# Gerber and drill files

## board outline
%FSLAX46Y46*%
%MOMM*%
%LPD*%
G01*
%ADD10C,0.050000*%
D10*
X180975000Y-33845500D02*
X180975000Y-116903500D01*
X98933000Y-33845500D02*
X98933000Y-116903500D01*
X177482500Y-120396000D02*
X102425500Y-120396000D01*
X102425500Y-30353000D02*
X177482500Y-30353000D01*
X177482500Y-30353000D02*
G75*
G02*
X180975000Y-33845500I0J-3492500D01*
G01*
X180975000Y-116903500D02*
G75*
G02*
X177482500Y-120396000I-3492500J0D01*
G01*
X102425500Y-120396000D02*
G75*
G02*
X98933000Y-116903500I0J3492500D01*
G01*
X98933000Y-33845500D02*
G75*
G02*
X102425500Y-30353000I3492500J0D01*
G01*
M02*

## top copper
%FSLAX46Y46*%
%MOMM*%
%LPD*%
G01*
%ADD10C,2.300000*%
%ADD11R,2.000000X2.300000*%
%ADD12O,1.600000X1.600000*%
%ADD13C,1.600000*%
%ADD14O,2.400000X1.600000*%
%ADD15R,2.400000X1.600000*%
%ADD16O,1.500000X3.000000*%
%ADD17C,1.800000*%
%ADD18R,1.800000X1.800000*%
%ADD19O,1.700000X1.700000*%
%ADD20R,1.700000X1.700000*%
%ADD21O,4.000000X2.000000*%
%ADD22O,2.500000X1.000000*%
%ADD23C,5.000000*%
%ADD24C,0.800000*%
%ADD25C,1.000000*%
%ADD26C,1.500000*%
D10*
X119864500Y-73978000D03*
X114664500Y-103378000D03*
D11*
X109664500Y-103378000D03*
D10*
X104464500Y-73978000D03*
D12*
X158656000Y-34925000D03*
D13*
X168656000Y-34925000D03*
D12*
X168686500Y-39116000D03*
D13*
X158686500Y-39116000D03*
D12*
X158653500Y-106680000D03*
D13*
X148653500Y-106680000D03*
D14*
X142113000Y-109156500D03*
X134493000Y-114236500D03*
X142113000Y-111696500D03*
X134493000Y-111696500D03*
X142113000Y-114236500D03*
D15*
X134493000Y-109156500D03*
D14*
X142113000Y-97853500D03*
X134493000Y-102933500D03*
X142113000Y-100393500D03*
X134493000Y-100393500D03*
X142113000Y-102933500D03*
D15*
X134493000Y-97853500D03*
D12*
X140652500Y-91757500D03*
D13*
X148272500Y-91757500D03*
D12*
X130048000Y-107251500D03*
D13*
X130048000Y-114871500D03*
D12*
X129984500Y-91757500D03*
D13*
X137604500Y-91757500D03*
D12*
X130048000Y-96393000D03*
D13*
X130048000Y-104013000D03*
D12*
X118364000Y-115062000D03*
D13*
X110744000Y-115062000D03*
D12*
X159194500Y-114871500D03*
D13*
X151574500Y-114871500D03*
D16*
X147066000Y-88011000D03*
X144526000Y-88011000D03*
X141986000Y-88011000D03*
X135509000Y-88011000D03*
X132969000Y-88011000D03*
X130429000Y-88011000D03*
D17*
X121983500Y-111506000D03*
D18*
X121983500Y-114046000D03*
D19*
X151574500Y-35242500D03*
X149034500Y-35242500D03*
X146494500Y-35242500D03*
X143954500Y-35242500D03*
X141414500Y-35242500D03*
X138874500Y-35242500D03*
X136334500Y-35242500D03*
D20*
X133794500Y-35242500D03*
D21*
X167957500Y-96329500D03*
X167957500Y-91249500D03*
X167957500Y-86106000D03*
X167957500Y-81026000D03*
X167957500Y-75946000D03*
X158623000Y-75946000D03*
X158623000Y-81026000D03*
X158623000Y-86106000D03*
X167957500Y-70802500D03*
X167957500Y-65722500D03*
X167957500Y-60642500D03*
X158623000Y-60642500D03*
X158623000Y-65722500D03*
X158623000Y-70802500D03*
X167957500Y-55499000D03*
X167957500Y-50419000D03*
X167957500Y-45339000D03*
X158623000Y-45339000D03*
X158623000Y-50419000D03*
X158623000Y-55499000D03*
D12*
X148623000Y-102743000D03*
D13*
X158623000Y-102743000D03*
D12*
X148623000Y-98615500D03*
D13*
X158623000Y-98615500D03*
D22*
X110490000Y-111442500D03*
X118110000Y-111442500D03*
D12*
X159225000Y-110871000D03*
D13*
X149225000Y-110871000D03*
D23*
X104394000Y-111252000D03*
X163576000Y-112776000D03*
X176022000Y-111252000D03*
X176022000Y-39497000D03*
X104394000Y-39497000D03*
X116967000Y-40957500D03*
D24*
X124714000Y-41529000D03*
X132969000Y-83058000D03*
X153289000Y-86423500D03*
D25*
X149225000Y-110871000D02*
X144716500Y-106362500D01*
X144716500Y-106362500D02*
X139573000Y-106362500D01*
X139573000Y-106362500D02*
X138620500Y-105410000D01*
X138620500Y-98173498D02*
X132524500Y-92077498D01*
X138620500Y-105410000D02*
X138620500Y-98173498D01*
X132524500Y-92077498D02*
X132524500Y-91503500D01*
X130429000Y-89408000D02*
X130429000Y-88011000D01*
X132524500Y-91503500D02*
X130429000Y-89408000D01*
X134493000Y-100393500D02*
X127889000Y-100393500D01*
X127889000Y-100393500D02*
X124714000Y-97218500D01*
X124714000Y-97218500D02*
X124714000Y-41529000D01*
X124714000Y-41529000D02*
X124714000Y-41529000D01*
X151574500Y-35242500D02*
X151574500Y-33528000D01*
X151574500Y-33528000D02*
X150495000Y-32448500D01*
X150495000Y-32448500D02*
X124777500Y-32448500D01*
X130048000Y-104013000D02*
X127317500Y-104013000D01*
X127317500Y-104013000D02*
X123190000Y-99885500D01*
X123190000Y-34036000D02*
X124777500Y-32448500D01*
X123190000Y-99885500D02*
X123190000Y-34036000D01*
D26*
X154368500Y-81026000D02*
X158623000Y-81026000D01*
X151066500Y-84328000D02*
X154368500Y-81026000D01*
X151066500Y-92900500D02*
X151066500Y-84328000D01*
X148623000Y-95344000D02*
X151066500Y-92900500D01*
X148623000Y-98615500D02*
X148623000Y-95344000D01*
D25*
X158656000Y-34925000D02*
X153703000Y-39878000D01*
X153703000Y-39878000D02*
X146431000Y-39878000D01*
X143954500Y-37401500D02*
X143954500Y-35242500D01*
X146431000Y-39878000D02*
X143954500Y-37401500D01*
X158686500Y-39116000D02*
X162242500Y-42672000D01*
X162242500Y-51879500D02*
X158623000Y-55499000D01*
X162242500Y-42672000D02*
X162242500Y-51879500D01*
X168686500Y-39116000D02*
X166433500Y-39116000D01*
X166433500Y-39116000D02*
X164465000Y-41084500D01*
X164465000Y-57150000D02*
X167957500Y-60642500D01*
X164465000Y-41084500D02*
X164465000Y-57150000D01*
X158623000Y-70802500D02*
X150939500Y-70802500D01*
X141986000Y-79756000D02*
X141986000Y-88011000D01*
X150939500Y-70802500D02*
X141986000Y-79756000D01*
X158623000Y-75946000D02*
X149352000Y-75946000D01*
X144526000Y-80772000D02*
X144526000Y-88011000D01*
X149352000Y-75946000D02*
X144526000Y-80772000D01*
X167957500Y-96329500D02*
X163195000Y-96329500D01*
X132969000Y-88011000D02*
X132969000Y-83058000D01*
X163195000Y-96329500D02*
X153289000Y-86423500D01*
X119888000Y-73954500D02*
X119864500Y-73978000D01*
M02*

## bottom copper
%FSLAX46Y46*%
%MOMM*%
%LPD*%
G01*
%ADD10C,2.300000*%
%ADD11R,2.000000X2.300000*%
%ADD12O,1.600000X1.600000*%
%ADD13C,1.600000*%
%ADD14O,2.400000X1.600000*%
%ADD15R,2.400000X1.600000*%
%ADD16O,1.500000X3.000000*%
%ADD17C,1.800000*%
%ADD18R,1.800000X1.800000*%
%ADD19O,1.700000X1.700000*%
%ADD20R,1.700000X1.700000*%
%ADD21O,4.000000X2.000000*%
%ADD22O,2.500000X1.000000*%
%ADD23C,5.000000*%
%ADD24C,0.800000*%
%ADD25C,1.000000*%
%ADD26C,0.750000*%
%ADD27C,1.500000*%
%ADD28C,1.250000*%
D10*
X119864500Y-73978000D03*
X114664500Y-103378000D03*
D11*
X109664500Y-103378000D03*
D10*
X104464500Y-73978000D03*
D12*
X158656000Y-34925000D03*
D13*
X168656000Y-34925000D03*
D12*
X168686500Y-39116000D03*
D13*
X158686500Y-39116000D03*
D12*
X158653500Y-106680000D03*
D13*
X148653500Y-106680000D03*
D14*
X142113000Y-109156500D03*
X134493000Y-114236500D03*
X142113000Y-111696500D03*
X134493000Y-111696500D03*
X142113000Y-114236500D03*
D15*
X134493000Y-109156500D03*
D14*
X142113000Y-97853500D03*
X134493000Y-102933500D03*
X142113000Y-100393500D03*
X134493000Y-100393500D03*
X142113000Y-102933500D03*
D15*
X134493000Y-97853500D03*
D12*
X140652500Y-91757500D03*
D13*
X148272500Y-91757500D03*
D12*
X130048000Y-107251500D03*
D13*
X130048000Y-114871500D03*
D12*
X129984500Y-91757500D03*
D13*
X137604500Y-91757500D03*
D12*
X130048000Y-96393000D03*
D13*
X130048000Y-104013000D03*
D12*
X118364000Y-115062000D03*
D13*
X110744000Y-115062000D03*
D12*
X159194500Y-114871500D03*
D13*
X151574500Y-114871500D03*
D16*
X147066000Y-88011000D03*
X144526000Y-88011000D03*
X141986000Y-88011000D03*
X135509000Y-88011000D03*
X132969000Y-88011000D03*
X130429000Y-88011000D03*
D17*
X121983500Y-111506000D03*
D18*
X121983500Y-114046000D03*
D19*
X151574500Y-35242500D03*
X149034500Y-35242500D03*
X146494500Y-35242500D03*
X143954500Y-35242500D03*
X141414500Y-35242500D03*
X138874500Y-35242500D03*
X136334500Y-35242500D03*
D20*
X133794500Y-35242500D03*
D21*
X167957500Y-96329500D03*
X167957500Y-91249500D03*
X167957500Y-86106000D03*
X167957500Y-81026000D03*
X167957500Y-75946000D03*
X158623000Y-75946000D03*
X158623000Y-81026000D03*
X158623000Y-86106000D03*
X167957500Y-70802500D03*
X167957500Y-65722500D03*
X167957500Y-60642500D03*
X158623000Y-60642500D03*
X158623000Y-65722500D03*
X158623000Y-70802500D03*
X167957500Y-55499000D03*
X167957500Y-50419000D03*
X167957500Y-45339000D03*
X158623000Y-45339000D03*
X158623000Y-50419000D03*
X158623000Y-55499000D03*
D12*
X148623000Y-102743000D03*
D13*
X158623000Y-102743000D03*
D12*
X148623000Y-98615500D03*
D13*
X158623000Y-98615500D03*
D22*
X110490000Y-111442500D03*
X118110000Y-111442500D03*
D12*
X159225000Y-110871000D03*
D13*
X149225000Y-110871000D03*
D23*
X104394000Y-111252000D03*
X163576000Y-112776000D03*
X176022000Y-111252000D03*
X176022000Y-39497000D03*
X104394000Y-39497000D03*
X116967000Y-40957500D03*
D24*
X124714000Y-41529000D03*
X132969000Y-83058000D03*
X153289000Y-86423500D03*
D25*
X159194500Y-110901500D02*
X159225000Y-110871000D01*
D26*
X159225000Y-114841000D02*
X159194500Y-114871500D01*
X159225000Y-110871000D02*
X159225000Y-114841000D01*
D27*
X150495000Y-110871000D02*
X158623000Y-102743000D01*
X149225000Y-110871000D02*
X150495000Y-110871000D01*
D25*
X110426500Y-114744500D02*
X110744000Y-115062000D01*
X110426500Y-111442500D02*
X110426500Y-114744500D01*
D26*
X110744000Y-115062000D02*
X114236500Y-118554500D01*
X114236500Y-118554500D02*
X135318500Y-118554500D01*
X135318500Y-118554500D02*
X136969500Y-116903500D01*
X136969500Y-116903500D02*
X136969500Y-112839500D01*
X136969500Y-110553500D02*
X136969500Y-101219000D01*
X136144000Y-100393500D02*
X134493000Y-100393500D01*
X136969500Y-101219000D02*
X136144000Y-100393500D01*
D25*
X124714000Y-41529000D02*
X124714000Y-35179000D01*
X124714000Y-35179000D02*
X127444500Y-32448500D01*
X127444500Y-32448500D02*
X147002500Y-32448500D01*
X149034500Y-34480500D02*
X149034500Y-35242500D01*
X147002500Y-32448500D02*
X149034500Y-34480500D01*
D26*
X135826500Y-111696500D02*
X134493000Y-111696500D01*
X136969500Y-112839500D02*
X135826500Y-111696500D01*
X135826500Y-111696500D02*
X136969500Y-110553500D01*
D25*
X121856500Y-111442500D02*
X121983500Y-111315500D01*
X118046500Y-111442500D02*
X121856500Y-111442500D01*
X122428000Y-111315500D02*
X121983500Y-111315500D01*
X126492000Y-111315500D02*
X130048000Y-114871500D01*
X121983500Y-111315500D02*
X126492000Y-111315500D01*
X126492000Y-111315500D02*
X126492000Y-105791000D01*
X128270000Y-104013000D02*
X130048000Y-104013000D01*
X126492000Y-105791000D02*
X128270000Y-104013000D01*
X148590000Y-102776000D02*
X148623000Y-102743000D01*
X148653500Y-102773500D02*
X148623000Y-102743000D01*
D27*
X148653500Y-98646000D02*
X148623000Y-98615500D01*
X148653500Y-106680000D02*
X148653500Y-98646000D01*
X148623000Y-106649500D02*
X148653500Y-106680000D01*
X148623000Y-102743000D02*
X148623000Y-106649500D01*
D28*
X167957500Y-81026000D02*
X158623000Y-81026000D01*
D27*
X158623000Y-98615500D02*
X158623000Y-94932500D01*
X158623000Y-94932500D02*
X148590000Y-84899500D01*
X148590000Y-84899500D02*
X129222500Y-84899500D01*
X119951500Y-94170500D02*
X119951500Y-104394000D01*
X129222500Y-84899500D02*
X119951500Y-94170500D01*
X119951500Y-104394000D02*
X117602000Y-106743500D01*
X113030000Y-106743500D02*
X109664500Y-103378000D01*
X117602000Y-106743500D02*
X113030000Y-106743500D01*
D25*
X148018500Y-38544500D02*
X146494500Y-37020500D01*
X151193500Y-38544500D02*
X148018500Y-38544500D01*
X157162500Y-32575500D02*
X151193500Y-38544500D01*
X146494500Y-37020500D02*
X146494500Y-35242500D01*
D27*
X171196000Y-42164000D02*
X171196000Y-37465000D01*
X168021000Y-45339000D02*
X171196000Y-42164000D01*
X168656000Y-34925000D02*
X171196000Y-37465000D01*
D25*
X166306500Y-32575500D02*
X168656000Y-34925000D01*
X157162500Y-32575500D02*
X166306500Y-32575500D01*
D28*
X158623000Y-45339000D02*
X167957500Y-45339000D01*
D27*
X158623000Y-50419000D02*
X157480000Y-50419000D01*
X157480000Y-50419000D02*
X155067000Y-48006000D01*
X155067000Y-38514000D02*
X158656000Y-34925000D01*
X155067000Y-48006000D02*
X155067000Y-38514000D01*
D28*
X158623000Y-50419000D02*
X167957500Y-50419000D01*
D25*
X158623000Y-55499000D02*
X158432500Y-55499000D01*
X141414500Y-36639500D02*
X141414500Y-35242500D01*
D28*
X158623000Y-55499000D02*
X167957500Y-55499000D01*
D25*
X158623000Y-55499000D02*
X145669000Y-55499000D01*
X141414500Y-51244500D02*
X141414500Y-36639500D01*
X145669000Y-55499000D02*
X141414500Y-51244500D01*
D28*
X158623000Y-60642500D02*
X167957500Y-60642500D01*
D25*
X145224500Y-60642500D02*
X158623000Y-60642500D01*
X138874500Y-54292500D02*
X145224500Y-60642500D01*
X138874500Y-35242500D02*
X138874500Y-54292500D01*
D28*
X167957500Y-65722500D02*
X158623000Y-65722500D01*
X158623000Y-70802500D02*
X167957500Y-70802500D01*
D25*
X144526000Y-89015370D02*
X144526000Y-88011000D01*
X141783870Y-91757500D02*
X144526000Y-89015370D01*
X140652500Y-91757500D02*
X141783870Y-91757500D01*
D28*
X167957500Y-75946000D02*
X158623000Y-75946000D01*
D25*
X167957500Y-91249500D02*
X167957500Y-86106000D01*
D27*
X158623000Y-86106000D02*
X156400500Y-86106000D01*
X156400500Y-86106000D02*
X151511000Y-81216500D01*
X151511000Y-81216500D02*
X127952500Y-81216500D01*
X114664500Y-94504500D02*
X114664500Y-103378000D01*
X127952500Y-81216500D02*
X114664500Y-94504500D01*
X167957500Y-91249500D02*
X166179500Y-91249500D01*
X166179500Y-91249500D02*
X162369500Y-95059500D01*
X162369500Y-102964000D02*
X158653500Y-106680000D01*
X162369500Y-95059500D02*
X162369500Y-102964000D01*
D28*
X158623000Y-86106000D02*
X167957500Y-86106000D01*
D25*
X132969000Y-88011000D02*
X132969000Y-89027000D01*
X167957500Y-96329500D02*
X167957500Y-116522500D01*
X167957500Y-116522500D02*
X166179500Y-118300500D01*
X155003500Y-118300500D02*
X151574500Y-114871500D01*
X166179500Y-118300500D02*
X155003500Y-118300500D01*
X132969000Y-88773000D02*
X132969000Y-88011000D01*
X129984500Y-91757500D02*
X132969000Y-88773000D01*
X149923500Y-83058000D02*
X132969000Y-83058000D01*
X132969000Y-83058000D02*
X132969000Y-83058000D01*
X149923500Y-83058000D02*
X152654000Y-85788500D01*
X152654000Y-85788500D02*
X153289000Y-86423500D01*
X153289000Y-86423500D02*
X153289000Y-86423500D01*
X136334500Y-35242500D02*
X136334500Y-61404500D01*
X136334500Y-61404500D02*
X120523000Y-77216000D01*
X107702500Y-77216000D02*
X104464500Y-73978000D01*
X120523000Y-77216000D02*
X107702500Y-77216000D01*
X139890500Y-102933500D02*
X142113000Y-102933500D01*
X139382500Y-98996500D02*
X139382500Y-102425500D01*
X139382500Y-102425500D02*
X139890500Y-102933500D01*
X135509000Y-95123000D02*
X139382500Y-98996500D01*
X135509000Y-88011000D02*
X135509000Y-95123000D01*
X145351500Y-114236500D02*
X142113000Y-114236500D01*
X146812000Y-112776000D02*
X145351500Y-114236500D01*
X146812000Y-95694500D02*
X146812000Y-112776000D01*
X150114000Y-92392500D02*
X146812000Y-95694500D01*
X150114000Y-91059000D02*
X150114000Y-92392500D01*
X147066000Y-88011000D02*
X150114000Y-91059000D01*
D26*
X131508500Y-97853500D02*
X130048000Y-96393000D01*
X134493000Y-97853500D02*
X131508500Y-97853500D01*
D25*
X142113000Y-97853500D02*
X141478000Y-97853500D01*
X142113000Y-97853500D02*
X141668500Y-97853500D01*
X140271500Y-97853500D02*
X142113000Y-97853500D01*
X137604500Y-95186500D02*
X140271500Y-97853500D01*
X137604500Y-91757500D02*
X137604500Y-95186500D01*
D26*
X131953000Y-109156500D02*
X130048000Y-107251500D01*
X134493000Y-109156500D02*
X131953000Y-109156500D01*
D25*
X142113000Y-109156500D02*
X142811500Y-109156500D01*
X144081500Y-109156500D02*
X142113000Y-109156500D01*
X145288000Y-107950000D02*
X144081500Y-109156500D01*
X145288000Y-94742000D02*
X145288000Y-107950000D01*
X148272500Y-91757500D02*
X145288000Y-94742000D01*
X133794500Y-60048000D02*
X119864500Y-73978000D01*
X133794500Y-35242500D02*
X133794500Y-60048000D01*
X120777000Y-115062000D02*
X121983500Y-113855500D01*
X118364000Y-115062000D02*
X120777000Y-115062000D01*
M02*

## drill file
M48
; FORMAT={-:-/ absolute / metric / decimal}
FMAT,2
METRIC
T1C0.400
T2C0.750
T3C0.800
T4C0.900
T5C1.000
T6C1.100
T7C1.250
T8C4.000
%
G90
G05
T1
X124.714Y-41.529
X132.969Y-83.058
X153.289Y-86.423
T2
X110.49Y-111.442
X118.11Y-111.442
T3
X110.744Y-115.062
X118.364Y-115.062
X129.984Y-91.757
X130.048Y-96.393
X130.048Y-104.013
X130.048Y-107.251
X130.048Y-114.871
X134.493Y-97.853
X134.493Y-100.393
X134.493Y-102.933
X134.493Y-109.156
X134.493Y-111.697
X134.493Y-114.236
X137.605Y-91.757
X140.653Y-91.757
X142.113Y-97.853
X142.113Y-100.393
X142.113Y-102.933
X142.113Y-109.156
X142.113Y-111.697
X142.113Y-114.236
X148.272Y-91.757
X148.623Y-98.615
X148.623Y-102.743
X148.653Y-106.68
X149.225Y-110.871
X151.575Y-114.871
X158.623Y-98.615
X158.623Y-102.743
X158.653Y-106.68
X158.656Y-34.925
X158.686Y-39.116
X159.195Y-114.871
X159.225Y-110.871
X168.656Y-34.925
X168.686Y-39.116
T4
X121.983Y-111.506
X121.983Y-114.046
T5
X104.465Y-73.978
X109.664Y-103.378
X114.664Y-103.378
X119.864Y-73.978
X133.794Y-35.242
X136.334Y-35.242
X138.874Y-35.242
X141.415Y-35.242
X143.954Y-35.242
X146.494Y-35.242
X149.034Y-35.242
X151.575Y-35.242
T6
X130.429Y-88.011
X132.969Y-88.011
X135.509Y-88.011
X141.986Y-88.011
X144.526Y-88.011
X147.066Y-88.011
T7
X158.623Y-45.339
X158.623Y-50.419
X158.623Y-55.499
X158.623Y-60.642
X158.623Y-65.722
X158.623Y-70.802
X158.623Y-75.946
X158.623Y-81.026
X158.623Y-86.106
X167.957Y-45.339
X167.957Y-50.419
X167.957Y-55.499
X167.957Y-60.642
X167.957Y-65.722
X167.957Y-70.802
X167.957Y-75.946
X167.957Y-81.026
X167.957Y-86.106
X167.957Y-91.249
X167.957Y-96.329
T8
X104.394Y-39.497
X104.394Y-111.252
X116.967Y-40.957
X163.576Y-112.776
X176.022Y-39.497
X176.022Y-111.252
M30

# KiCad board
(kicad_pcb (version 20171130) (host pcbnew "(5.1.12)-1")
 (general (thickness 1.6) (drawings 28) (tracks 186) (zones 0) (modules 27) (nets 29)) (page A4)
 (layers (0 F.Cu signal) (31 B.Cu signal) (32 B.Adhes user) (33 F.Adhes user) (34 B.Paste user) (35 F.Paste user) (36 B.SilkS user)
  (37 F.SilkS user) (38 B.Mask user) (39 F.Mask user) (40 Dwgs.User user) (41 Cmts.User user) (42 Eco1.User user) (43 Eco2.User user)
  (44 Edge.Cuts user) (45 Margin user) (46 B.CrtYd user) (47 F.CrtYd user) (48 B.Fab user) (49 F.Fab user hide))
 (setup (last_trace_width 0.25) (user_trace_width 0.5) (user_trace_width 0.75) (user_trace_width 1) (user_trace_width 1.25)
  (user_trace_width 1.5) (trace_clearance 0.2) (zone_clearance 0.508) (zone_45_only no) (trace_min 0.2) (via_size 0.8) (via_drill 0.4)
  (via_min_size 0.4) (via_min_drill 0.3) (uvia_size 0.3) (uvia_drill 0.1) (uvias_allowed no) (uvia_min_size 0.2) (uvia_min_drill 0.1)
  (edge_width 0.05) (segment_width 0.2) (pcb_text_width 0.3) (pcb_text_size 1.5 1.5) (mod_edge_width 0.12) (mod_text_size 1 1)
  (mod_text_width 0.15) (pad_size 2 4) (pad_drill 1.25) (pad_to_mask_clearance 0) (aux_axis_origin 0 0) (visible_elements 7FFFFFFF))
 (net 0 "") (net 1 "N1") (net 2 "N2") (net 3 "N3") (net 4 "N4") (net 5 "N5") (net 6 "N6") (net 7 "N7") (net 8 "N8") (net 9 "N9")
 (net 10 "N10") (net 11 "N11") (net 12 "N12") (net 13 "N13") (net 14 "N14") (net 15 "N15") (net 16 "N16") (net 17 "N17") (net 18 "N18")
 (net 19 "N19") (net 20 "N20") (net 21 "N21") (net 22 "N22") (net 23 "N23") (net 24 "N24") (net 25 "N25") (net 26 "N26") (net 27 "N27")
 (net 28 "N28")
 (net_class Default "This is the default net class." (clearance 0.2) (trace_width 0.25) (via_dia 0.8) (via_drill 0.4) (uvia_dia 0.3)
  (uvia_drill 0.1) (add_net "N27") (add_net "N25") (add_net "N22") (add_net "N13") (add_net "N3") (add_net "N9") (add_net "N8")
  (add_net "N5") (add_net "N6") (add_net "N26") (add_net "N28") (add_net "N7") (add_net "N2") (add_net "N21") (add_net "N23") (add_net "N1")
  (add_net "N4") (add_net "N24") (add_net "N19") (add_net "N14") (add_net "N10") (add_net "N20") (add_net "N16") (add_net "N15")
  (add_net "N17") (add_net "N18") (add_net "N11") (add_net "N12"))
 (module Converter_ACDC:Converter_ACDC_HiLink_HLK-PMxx (layer F.Cu) (at 109.6645 103.378 90)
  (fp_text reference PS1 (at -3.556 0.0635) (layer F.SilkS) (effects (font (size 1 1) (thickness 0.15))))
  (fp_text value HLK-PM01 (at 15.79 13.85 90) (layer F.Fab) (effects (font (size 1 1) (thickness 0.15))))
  (pad 4 thru_hole circle (at 29.4 10.2 90) (size 2.3 2.3) (drill 1) (layers *.Cu *.Mask) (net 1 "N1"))
  (pad 2 thru_hole circle (at 0 5 90) (size 2.3 2.3) (drill 1) (layers *.Cu *.Mask) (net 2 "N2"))
  (pad 1 thru_hole rect (at 0 0 90) (size 2.3 2) (drill 1) (layers *.Cu *.Mask) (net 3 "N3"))
  (pad 3 thru_hole circle (at 29.4 -5.2 90) (size 2.3 2.3) (drill 1) (layers *.Cu *.Mask) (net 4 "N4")))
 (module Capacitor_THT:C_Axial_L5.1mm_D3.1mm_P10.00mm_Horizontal (layer F.Cu) (at 168.656 34.925 180)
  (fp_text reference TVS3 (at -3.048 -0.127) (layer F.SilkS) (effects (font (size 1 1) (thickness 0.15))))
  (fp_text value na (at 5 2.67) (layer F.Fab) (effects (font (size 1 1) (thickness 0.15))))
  (pad 2 thru_hole oval (at 10 0 180) (size 1.6 1.6) (drill 0.8) (layers *.Cu *.Mask) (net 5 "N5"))
  (pad 1 thru_hole circle (at 0 0 180) (size 1.6 1.6) (drill 0.8) (layers *.Cu *.Mask) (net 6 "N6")))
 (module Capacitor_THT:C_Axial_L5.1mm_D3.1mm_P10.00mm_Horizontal (layer F.Cu) (at 158.6865 39.116)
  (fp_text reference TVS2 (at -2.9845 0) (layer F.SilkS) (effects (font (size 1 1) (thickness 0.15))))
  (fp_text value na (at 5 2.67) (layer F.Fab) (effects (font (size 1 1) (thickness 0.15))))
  (pad 2 thru_hole oval (at 10 0) (size 1.6 1.6) (drill 0.8) (layers *.Cu *.Mask) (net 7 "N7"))
  (pad 1 thru_hole circle (at 0 0) (size 1.6 1.6) (drill 0.8) (layers *.Cu *.Mask) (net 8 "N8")))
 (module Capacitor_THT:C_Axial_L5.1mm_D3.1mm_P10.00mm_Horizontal (layer F.Cu) (at 148.6535 106.68)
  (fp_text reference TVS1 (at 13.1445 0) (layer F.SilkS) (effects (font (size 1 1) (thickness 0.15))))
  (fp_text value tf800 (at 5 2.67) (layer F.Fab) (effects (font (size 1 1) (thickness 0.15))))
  (pad 2 thru_hole oval (at 10 0) (size 1.6 1.6) (drill 0.8) (layers *.Cu *.Mask) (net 2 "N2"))
  (pad 1 thru_hole circle (at 0 0) (size 1.6 1.6) (drill 0.8) (layers *.Cu *.Mask) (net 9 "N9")))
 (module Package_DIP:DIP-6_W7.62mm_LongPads (layer F.Cu) (at 134.493 109.1565)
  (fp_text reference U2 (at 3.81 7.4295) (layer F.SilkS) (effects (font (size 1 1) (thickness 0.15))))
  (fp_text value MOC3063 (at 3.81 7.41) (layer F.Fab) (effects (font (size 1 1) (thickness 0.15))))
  (pad 6 thru_hole oval (at 7.62 0) (size 2.4 1.6) (drill 0.8) (layers *.Cu *.Mask) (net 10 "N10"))
  (pad 3 thru_hole oval (at 0 5.08) (size 2.4 1.6) (drill 0.8) (layers *.Cu *.Mask) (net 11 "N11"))
  (pad 5 thru_hole oval (at 7.62 2.54) (size 2.4 1.6) (drill 0.8) (layers *.Cu *.Mask) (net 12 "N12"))
  (pad 2 thru_hole oval (at 0 2.54) (size 2.4 1.6) (drill 0.8) (layers *.Cu *.Mask) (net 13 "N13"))
  (pad 4 thru_hole oval (at 7.62 5.08) (size 2.4 1.6) (drill 0.8) (layers *.Cu *.Mask) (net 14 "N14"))
  (pad 1 thru_hole rect (at 0 0) (size 2.4 1.6) (drill 0.8) (layers *.Cu *.Mask) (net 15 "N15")))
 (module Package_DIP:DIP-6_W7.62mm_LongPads (layer F.Cu) (at 134.493 97.8535)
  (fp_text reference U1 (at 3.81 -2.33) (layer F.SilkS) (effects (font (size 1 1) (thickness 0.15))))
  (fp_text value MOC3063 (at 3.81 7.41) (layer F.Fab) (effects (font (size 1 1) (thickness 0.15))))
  (pad 6 thru_hole oval (at 7.62 0) (size 2.4 1.6) (drill 0.8) (layers *.Cu *.Mask) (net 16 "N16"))
  (pad 3 thru_hole oval (at 0 5.08) (size 2.4 1.6) (drill 0.8) (layers *.Cu *.Mask) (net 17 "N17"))
  (pad 5 thru_hole oval (at 7.62 2.54) (size 2.4 1.6) (drill 0.8) (layers *.Cu *.Mask) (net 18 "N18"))
  (pad 2 thru_hole oval (at 0 2.54) (size 2.4 1.6) (drill 0.8) (layers *.Cu *.Mask) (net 13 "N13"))
  (pad 4 thru_hole oval (at 7.62 5.08) (size 2.4 1.6) (drill 0.8) (layers *.Cu *.Mask) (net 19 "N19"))
  (pad 1 thru_hole rect (at 0 0) (size 2.4 1.6) (drill 0.8) (layers *.Cu *.Mask) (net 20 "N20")))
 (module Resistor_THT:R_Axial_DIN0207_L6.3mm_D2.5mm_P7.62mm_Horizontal (layer F.Cu) (at 148.2725 91.7575 180)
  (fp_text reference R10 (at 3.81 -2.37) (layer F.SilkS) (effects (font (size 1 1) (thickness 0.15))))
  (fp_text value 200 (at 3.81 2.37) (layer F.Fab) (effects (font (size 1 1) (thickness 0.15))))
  (pad 2 thru_hole oval (at 7.62 0 180) (size 1.6 1.6) (drill 0.8) (layers *.Cu *.Mask) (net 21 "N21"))
  (pad 1 thru_hole circle (at 0 0 180) (size 1.6 1.6) (drill 0.8) (layers *.Cu *.Mask) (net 10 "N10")))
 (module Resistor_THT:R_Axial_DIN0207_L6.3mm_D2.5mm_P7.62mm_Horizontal (layer F.Cu) (at 130.048 114.8715 90)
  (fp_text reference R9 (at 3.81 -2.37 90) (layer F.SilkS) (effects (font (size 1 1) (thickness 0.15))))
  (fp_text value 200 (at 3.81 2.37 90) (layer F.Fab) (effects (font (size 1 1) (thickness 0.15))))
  (pad 2 thru_hole oval (at 7.62 0 90) (size 1.6 1.6) (drill 0.8) (layers *.Cu *.Mask) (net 15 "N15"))
  (pad 1 thru_hole circle (at 0 0 90) (size 1.6 1.6) (drill 0.8) (layers *.Cu *.Mask) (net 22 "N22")))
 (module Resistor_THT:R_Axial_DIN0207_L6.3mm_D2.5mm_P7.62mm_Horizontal (layer F.Cu) (at 137.6045 91.7575 180)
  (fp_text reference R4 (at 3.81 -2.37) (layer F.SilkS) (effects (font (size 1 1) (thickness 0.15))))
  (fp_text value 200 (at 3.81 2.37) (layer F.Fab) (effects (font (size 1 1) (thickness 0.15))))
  (pad 2 thru_hole oval (at 7.62 0 180) (size 1.6 1.6) (drill 0.8) (layers *.Cu *.Mask) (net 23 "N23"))
  (pad 1 thru_hole circle (at 0 0 180) (size 1.6 1.6) (drill 0.8) (layers *.Cu *.Mask) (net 16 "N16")))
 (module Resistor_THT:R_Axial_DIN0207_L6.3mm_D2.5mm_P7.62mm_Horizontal (layer F.Cu) (at 130.048 104.013 90)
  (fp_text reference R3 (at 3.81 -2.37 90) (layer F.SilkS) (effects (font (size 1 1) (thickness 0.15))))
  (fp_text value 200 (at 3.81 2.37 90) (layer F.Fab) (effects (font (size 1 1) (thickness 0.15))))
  (pad 2 thru_hole oval (at 7.62 0 90) (size 1.6 1.6) (drill 0.8) (layers *.Cu *.Mask) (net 20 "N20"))
  (pad 1 thru_hole circle (at 0 0 90) (size 1.6 1.6) (drill 0.8) (layers *.Cu *.Mask) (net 22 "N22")))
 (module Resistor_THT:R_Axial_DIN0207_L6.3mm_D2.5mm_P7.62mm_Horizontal (layer F.Cu) (at 110.744 115.062)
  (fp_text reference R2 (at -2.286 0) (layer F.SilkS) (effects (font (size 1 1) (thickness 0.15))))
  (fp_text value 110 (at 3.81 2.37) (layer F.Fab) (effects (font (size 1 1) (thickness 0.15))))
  (pad 2 thru_hole oval (at 7.62 0) (size 1.6 1.6) (drill 0.8) (layers *.Cu *.Mask) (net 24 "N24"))
  (pad 1 thru_hole circle (at 0 0) (size 1.6 1.6) (drill 0.8) (layers *.Cu *.Mask) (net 13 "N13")))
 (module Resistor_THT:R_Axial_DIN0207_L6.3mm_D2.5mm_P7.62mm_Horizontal (layer F.Cu) (at 151.5745 114.8715)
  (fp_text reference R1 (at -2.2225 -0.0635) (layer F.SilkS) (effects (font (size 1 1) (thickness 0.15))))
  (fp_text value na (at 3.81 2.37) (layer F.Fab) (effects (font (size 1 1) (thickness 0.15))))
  (pad 2 thru_hole oval (at 7.62 0) (size 1.6 1.6) (drill 0.8) (layers *.Cu *.Mask) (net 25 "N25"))
  (pad 1 thru_hole circle (at 0 0) (size 1.6 1.6) (drill 0.8) (layers *.Cu *.Mask) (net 23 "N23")))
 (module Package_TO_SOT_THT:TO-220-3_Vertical (layer F.Cu) (at 141.986 88.011)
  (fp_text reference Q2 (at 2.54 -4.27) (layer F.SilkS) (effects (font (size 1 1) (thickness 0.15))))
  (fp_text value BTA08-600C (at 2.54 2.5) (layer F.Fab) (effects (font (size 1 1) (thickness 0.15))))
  (pad 3 thru_hole oval (at 5.08 0) (size 1.5 3) (drill 1.1) (layers *.Cu *.Mask) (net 14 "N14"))
  (pad 2 thru_hole oval (at 2.54 0) (size 1.5 3) (drill 1.1) (layers *.Cu *.Mask) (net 21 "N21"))
  (pad 1 thru_hole oval (at 0 0) (size 1.5 3) (drill 1.1) (layers *.Cu *.Mask) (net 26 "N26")))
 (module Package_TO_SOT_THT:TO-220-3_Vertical (layer F.Cu) (at 130.429 88.011)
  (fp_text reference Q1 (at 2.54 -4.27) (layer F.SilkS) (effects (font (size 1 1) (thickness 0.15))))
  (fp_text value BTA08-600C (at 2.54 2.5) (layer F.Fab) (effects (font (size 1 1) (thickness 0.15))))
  (pad 3 thru_hole oval (at 5.08 0) (size 1.5 3) (drill 1.1) (layers *.Cu *.Mask) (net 19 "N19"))
  (pad 2 thru_hole oval (at 2.54 0) (size 1.5 3) (drill 1.1) (layers *.Cu *.Mask) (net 23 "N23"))
  (pad 1 thru_hole oval (at 0 0) (size 1.5 3) (drill 1.1) (layers *.Cu *.Mask) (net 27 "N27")))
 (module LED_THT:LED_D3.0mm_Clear (layer F.Cu) (at 121.9835 114.046 90)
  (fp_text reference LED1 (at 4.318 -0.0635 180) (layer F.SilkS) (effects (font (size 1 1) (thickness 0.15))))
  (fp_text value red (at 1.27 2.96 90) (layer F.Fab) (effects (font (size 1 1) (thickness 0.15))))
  (pad 2 thru_hole circle (at 2.54 0 90) (size 1.8 1.8) (drill 0.9) (layers *.Cu *.Mask) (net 22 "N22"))
  (pad 1 thru_hole rect (at 0 0 90) (size 1.8 1.8) (drill 0.9) (layers *.Cu *.Mask) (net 24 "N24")))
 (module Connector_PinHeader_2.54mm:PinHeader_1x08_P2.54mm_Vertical (layer F.Cu) (at 133.7945 35.2425 90)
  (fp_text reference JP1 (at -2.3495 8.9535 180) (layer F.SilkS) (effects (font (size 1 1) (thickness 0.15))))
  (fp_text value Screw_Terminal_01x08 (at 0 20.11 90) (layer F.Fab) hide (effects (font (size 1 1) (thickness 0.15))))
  (pad 8 thru_hole oval (at 0 17.78 90) (size 1.7 1.7) (drill 1) (layers *.Cu *.Mask) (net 22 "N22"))
  (pad 7 thru_hole oval (at 0 15.24 90) (size 1.7 1.7) (drill 1) (layers *.Cu *.Mask) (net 13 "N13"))
  (pad 6 thru_hole oval (at 0 12.7 90) (size 1.7 1.7) (drill 1) (layers *.Cu *.Mask) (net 6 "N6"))
  (pad 5 thru_hole oval (at 0 10.16 90) (size 1.7 1.7) (drill 1) (layers *.Cu *.Mask) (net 5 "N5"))
  (pad 4 thru_hole oval (at 0 7.62 90) (size 1.7 1.7) (drill 1) (layers *.Cu *.Mask) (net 8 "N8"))
  (pad 3 thru_hole oval (at 0 5.08 90) (size 1.7 1.7) (drill 1) (layers *.Cu *.Mask) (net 7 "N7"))
  (pad 2 thru_hole oval (at 0 2.54 90) (size 1.7 1.7) (drill 1) (layers *.Cu *.Mask) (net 4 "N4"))
  (pad 1 thru_hole rect (at 0 0 90) (size 1.7 1.7) (drill 1) (layers *.Cu *.Mask) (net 1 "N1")))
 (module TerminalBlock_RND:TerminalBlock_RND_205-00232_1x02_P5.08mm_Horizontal (layer F.Cu) (at 167.9575 91.2495 270)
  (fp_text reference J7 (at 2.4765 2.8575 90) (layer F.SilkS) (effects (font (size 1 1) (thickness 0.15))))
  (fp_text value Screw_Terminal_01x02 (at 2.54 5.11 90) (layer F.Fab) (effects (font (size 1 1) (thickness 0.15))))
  (pad 2 thru_hole oval (at 5.08 0 270) (size 2 4) (drill 1.25) (layers *.Cu *.Mask) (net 23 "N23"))
  (pad 1 thru_hole oval (at 0 0 270) (size 2 4) (drill 1.25) (layers *.Cu *.Mask) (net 2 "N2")))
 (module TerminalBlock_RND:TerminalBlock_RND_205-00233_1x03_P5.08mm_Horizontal (layer F.Cu) (at 167.9575 75.946 270)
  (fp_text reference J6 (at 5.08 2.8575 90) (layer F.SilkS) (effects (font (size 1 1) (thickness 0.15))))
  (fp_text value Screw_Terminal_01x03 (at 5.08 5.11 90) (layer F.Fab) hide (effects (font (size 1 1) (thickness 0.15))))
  (pad 3 thru_hole oval (at 10.16 0 270) (size 2 4) (drill 1.25) (layers *.Cu *.Mask) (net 2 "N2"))
  (pad 2 thru_hole oval (at 5.08 0 270) (size 2 4) (drill 1.25) (layers *.Cu *.Mask) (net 9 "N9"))
  (pad 1 thru_hole oval (at 0 0 270) (size 2 4) (drill 1.25) (layers *.Cu *.Mask) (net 21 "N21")))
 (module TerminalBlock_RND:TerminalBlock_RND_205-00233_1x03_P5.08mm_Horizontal (layer F.Cu) (at 158.623 86.106 90)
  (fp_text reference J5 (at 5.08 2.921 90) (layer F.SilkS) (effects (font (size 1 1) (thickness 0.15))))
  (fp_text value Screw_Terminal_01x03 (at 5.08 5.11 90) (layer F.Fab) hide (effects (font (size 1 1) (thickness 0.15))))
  (pad 3 thru_hole oval (at 10.16 0 90) (size 2 4) (drill 1.25) (layers *.Cu *.Mask) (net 21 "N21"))
  (pad 2 thru_hole oval (at 5.08 0 90) (size 2 4) (drill 1.25) (layers *.Cu *.Mask) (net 9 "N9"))
  (pad 1 thru_hole oval (at 0 0 90) (size 2 4) (drill 1.25) (layers *.Cu *.Mask) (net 2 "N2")))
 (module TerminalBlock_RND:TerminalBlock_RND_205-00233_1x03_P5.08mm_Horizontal (layer F.Cu) (at 167.9575 60.6425 270)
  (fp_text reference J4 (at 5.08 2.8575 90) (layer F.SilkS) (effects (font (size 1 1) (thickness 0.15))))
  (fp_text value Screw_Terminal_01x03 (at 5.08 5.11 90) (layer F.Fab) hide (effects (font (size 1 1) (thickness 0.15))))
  (pad 3 thru_hole oval (at 10.16 0 270) (size 2 4) (drill 1.25) (layers *.Cu *.Mask) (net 26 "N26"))
  (pad 2 thru_hole oval (at 5.08 0 270) (size 2 4) (drill 1.25) (layers *.Cu *.Mask) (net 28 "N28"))
  (pad 1 thru_hole oval (at 0 0 270) (size 2 4) (drill 1.25) (layers *.Cu *.Mask) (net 7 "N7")))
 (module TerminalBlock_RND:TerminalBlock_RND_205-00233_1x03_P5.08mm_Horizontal (layer F.Cu) (at 158.623 70.8025 90)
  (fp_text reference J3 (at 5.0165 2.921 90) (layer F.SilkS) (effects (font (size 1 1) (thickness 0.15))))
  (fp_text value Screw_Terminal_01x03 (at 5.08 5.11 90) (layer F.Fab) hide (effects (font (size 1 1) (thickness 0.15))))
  (pad 3 thru_hole oval (at 10.16 0 90) (size 2 4) (drill 1.25) (layers *.Cu *.Mask) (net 7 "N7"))
  (pad 2 thru_hole oval (at 5.08 0 90) (size 2 4) (drill 1.25) (layers *.Cu *.Mask) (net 28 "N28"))
  (pad 1 thru_hole oval (at 0 0 90) (size 2 4) (drill 1.25) (layers *.Cu *.Mask) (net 26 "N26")))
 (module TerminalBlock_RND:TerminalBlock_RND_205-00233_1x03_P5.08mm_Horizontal (layer F.Cu) (at 167.9575 45.339 270)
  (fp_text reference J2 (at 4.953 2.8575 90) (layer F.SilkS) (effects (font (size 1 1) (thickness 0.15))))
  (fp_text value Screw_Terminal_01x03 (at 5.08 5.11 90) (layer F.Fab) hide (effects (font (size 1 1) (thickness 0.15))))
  (pad 3 thru_hole oval (at 10.16 0 270) (size 2 4) (drill 1.25) (layers *.Cu *.Mask) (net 8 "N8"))
  (pad 2 thru_hole oval (at 5.08 0 270) (size 2 4) (drill 1.25) (layers *.Cu *.Mask) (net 5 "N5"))
  (pad 1 thru_hole oval (at 0 0 270) (size 2 4) (drill 1.25) (layers *.Cu *.Mask) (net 6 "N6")))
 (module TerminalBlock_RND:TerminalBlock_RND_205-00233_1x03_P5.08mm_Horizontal (layer F.Cu) (at 158.623 55.499 90)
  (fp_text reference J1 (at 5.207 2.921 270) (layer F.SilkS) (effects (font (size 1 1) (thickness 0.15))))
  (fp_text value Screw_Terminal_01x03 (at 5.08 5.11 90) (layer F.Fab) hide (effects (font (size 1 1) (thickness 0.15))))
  (pad 3 thru_hole oval (at 10.16 0 90) (size 2 4) (drill 1.25) (layers *.Cu *.Mask) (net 6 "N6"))
  (pad 2 thru_hole oval (at 5.08 0 90) (size 2 4) (drill 1.25) (layers *.Cu *.Mask) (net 5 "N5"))
  (pad 1 thru_hole oval (at 0 0 90) (size 2 4) (drill 1.25) (layers *.Cu *.Mask) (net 8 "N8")))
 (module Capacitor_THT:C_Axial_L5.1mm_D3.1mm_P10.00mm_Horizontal (layer F.Cu) (at 158.623 102.743 180)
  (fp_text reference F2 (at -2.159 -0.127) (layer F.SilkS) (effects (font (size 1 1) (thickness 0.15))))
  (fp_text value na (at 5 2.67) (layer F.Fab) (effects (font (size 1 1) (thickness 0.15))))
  (pad 2 thru_hole oval (at 10 0 180) (size 1.6 1.6) (drill 0.8) (layers *.Cu *.Mask) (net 9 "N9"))
  (pad 1 thru_hole circle (at 0 0 180) (size 1.6 1.6) (drill 0.8) (layers *.Cu *.Mask) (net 27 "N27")))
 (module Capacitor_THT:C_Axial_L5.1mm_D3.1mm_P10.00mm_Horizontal (layer F.Cu) (at 158.623 98.6155 180)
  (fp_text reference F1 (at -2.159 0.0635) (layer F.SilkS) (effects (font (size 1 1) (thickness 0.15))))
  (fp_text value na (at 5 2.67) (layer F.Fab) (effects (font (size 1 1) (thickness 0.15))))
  (pad 2 thru_hole oval (at 10 0 180) (size 1.6 1.6) (drill 0.8) (layers *.Cu *.Mask) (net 9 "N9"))
  (pad 1 thru_hole circle (at 0 0 180) (size 1.6 1.6) (drill 0.8) (layers *.Cu *.Mask) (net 3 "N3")))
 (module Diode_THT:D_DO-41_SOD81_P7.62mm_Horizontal (layer F.Cu) (at 118.11 111.4425 180)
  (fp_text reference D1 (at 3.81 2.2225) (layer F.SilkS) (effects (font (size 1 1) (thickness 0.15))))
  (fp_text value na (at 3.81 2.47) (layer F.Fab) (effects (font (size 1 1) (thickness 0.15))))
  (pad 2 thru_hole oval (at 7.62 0 180) (size 2.5 1) (drill 0.75) (layers *.Cu *.Mask) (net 13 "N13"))
  (pad 1 thru_hole oval (at 0 0 180) (size 2.5 1) (drill 0.75) (layers *.Cu *.Mask) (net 22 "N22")))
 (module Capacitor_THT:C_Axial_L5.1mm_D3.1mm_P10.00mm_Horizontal (layer F.Cu) (at 149.225 110.871)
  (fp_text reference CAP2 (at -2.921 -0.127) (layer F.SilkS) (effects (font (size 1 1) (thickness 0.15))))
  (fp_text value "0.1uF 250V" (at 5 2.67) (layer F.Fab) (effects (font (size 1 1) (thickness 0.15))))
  (pad 2 thru_hole oval (at 10 0) (size 1.6 1.6) (drill 0.8) (layers *.Cu *.Mask) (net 25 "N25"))
  (pad 1 thru_hole circle (at 0 0) (size 1.6 1.6) (drill 0.8) (layers *.Cu *.Mask) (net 27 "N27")))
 (gr_line (start 180.975 33.8455) (end 180.975 116.9035) (layer Edge.Cuts) (width 0.05))
 (gr_line (start 98.933 33.8455) (end 98.933 116.9035) (layer Edge.Cuts) (width 0.05))
 (gr_line (start 177.4825 120.396) (end 102.4255 120.396) (layer Edge.Cuts) (width 0.05))
 (gr_line (start 102.4255 30.353) (end 177.4825 30.353) (layer Edge.Cuts) (width 0.05))
 (gr_arc (start 177.4825 33.8455) (end 180.975 33.8455) (angle -90) (layer Edge.Cuts) (width 0.05))
 (gr_arc (start 177.4825 116.9035) (end 177.4825 120.396) (angle -90) (layer Edge.Cuts) (width 0.05))
 (gr_arc (start 102.4255 116.9035) (end 98.933 116.9035) (angle -90) (layer Edge.Cuts) (width 0.05))
 (gr_arc (start 102.4255 33.8455) (end 102.4255 30.353) (angle -90) (layer Edge.Cuts) (width 0.05))
 (via (at 104.394 111.252) (size 5) (drill 4) (layers F.Cu B.Cu) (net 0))
 (via (at 163.576 112.776) (size 5) (drill 4) (layers F.Cu B.Cu) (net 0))
 (via (at 176.022 111.252) (size 5) (drill 4) (layers F.Cu B.Cu) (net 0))
 (via (at 176.022 39.497) (size 5) (drill 4) (layers F.Cu B.Cu) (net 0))
 (via (at 104.394 39.497) (size 5) (drill 4) (layers F.Cu B.Cu) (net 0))
 (via (at 116.967 40.9575) (size 5) (drill 4) (layers F.Cu B.Cu) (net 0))
 (segment (start 159.1945 110.9015) (end 159.225 110.871) (width 1) (layer B.Cu) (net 25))
 (segment (start 159.225 114.841) (end 159.1945 114.8715) (width 0.75) (layer B.Cu) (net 25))
 (segment (start 159.225 110.871) (end 159.225 114.841) (width 0.75) (layer B.Cu) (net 25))
 (segment (start 150.495 110.871) (end 158.623 102.743) (width 1.5) (layer B.Cu) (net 27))
 (segment (start 149.225 110.871) (end 150.495 110.871) (width 1.5) (layer B.Cu) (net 27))
 (segment (start 149.225 110.871) (end 144.7165 106.3625) (width 1) (layer F.Cu) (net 27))
 (segment (start 144.7165 106.3625) (end 139.573 106.3625) (width 1) (layer F.Cu) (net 27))
 (segment (start 139.573 106.3625) (end 138.6205 105.41) (width 1) (layer F.Cu) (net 27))
 (segment (start 138.6205 98.173498) (end 132.5245 92.077498) (width 1) (layer F.Cu) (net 27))
 (segment (start 138.6205 105.41) (end 138.6205 98.173498) (width 1) (layer F.Cu) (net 27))
 (segment (start 132.5245 92.077498) (end 132.5245 91.5035) (width 1) (layer F.Cu) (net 27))
 (segment (start 130.429 89.408) (end 130.429 88.011) (width 1) (layer F.Cu) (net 27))
 (segment (start 132.5245 91.5035) (end 130.429 89.408) (width 1) (layer F.Cu) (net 27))
 (segment (start 110.4265 114.7445) (end 110.744 115.062) (width 1) (layer B.Cu) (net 13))
 (segment (start 110.4265 111.4425) (end 110.4265 114.7445) (width 1) (layer B.Cu) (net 13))
 (segment (start 134.493 100.3935) (end 127.889 100.3935) (width 1) (layer F.Cu) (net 13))
 (segment (start 127.889 100.3935) (end 124.714 97.2185) (width 1) (layer F.Cu) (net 13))
 (segment (start 124.714 97.2185) (end 124.714 41.529) (width 1) (layer F.Cu) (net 13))
 (segment (start 110.744 115.062) (end 114.2365 118.5545) (width 0.75) (layer B.Cu) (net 13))
 (segment (start 114.2365 118.5545) (end 135.3185 118.5545) (width 0.75) (layer B.Cu) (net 13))
 (segment (start 135.3185 118.5545) (end 136.9695 116.9035) (width 0.75) (layer B.Cu) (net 13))
 (segment (start 136.9695 116.9035) (end 136.9695 112.8395) (width 0.75) (layer B.Cu) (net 13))
 (segment (start 136.9695 110.5535) (end 136.9695 101.219) (width 0.75) (layer B.Cu) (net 13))
 (segment (start 136.144 100.3935) (end 134.493 100.3935) (width 0.75) (layer B.Cu) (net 13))
 (segment (start 136.9695 101.219) (end 136.144 100.3935) (width 0.75) (layer B.Cu) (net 13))
 (segment (start 124.714 41.529) (end 124.714 41.529) (width 1) (layer F.Cu) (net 13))
 (via (at 124.714 41.529) (size 0.8) (drill 0.4) (layers F.Cu B.Cu) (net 13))
 (segment (start 124.714 41.529) (end 124.714 35.179) (width 1) (layer B.Cu) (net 13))
 (segment (start 124.714 35.179) (end 127.4445 32.4485) (width 1) (layer B.Cu) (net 13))
 (segment (start 127.4445 32.4485) (end 147.0025 32.4485) (width 1) (layer B.Cu) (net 13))
 (segment (start 149.0345 34.4805) (end 149.0345 35.2425) (width 1) (layer B.Cu) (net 13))
 (segment (start 147.0025 32.4485) (end 149.0345 34.4805) (width 1) (layer B.Cu) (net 13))
 (segment (start 135.8265 111.6965) (end 134.493 111.6965) (width 0.75) (layer B.Cu) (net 13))
 (segment (start 136.9695 112.8395) (end 135.8265 111.6965) (width 0.75) (layer B.Cu) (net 13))
 (segment (start 135.8265 111.6965) (end 136.9695 110.5535) (width 0.75) (layer B.Cu) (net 13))
 (segment (start 121.8565 111.4425) (end 121.9835 111.3155) (width 1) (layer B.Cu) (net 22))
 (segment (start 118.0465 111.4425) (end 121.8565 111.4425) (width 1) (layer B.Cu) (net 22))
 (segment (start 122.428 111.3155) (end 121.9835 111.3155) (width 1) (layer B.Cu) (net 22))
 (segment (start 151.5745 35.2425) (end 151.5745 33.528) (width 1) (layer F.Cu) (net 22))
 (segment (start 151.5745 33.528) (end 150.495 32.4485) (width 1) (layer F.Cu) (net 22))
 (segment (start 150.495 32.4485) (end 124.7775 32.4485) (width 1) (layer F.Cu) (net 22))
 (segment (start 130.048 104.013) (end 127.3175 104.013) (width 1) (layer F.Cu) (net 22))
 (segment (start 127.3175 104.013) (end 123.19 99.8855) (width 1) (layer F.Cu) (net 22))
 (segment (start 123.19 34.036) (end 124.7775 32.4485) (width 1) (layer F.Cu) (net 22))
 (segment (start 123.19 99.8855) (end 123.19 34.036) (width 1) (layer F.Cu) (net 22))
 (segment (start 126.492 111.3155) (end 130.048 114.8715) (width 1) (layer B.Cu) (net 22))
 (segment (start 121.9835 111.3155) (end 126.492 111.3155) (width 1) (layer B.Cu) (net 22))
 (segment (start 126.492 111.3155) (end 126.492 105.791) (width 1) (layer B.Cu) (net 22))
 (segment (start 128.27 104.013) (end 130.048 104.013) (width 1) (layer B.Cu) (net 22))
 (segment (start 126.492 105.791) (end 128.27 104.013) (width 1) (layer B.Cu) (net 22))
 (segment (start 148.59 102.776) (end 148.623 102.743) (width 1) (layer B.Cu) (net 9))
 (segment (start 148.6535 102.7735) (end 148.623 102.743) (width 1) (layer B.Cu) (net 9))
 (segment (start 148.6535 98.646) (end 148.623 98.6155) (width 1.5) (layer B.Cu) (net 9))
 (segment (start 148.6535 106.68) (end 148.6535 98.646) (width 1.5) (layer B.Cu) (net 9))
 (segment (start 148.623 106.6495) (end 148.6535 106.68) (width 1.5) (layer B.Cu) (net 9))
 (segment (start 148.623 102.743) (end 148.623 106.6495) (width 1.5) (layer B.Cu) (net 9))
 (segment (start 154.3685 81.026) (end 158.623 81.026) (width 1.5) (layer F.Cu) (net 9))
 (segment (start 151.0665 84.328) (end 154.3685 81.026) (width 1.5) (layer F.Cu) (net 9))
 (segment (start 151.0665 92.9005) (end 151.0665 84.328) (width 1.5) (layer F.Cu) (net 9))
 (segment (start 148.623 95.344) (end 151.0665 92.9005) (width 1.5) (layer F.Cu) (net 9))
 (segment (start 148.623 98.6155) (end 148.623 95.344) (width 1.5) (layer F.Cu) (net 9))
 (segment (start 167.9575 81.026) (end 158.623 81.026) (width 1.25) (layer B.Cu) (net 9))
 (segment (start 158.623 98.6155) (end 158.623 94.9325) (width 1.5) (layer B.Cu) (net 3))
 (segment (start 158.623 94.9325) (end 148.59 84.8995) (width 1.5) (layer B.Cu) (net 3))
 (segment (start 148.59 84.8995) (end 129.2225 84.8995) (width 1.5) (layer B.Cu) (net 3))
 (segment (start 119.9515 94.1705) (end 119.9515 104.394) (width 1.5) (layer B.Cu) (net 3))
 (segment (start 129.2225 84.8995) (end 119.9515 94.1705) (width 1.5) (layer B.Cu) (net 3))
 (segment (start 119.9515 104.394) (end 117.602 106.7435) (width 1.5) (layer B.Cu) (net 3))
 (segment (start 113.03 106.7435) (end 109.6645 103.378) (width 1.5) (layer B.Cu) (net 3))
 (segment (start 117.602 106.7435) (end 113.03 106.7435) (width 1.5) (layer B.Cu) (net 3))
 (segment (start 148.0185 38.5445) (end 146.4945 37.0205) (width 1) (layer B.Cu) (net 6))
 (segment (start 151.1935 38.5445) (end 148.0185 38.5445) (width 1) (layer B.Cu) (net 6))
 (segment (start 157.1625 32.5755) (end 151.1935 38.5445) (width 1) (layer B.Cu) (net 6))
 (segment (start 146.4945 37.0205) (end 146.4945 35.2425) (width 1) (layer B.Cu) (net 6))
 (segment (start 171.196 42.164) (end 171.196 37.465) (width 1.5) (layer B.Cu) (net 6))
 (segment (start 168.021 45.339) (end 171.196 42.164) (width 1.5) (layer B.Cu) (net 6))
 (segment (start 168.656 34.925) (end 171.196 37.465) (width 1.5) (layer B.Cu) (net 6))
 (segment (start 166.3065 32.5755) (end 168.656 34.925) (width 1) (layer B.Cu) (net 6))
 (segment (start 157.1625 32.5755) (end 166.3065 32.5755) (width 1) (layer B.Cu) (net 6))
 (segment (start 158.623 45.339) (end 167.9575 45.339) (width 1.25) (layer B.Cu) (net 6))
 (segment (start 158.656 34.925) (end 153.703 39.878) (width 1) (layer F.Cu) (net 5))
 (segment (start 153.703 39.878) (end 146.431 39.878) (width 1) (layer F.Cu) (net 5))
 (segment (start 143.9545 37.4015) (end 143.9545 35.2425) (width 1) (layer F.Cu) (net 5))
 (segment (start 146.431 39.878) (end 143.9545 37.4015) (width 1) (layer F.Cu) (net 5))
 (segment (start 158.623 50.419) (end 157.48 50.419) (width 1.5) (layer B.Cu) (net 5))
 (segment (start 157.48 50.419) (end 155.067 48.006) (width 1.5) (layer B.Cu) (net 5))
 (segment (start 155.067 38.514) (end 158.656 34.925) (width 1.5) (layer B.Cu) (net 5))
 (segment (start 155.067 48.006) (end 155.067 38.514) (width 1.5) (layer B.Cu) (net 5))
 (segment (start 158.623 50.419) (end 167.9575 50.419) (width 1.25) (layer B.Cu) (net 5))
 (segment (start 158.6865 39.116) (end 162.2425 42.672) (width 1) (layer F.Cu) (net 8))
 (segment (start 158.623 55.499) (end 158.4325 55.499) (width 1) (layer B.Cu) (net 8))
 (segment (start 141.4145 36.6395) (end 141.4145 35.2425) (width 1) (layer B.Cu) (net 8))
 (segment (start 158.623 55.499) (end 167.9575 55.499) (width 1.25) (layer B.Cu) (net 8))
 (segment (start 162.2425 51.8795) (end 158.623 55.499) (width 1) (layer F.Cu) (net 8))
 (segment (start 162.2425 42.672) (end 162.2425 51.8795) (width 1) (layer F.Cu) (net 8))
 (segment (start 158.623 55.499) (end 145.669 55.499) (width 1) (layer B.Cu) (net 8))
 (segment (start 141.4145 51.2445) (end 141.4145 36.6395) (width 1) (layer B.Cu) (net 8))
 (segment (start 145.669 55.499) (end 141.4145 51.2445) (width 1) (layer B.Cu) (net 8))
 (segment (start 168.6865 39.116) (end 166.4335 39.116) (width 1) (layer F.Cu) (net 7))
 (segment (start 166.4335 39.116) (end 164.465 41.0845) (width 1) (layer F.Cu) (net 7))
 (segment (start 158.623 60.6425) (end 167.9575 60.6425) (width 1.25) (layer B.Cu) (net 7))
 (segment (start 164.465 57.15) (end 167.9575 60.6425) (width 1) (layer F.Cu) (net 7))
 (segment (start 164.465 41.0845) (end 164.465 57.15) (width 1) (layer F.Cu) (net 7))
 (segment (start 145.2245 60.6425) (end 158.623 60.6425) (width 1) (layer B.Cu) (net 7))
 (segment (start 138.8745 54.2925) (end 145.2245 60.6425) (width 1) (layer B.Cu) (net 7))
 (segment (start 138.8745 35.2425) (end 138.8745 54.2925) (width 1) (layer B.Cu) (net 7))
 (segment (start 167.9575 65.7225) (end 158.623 65.7225) (width 1.25) (layer B.Cu) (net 28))
 (segment (start 158.623 70.8025) (end 150.9395 70.8025) (width 1) (layer F.Cu) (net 26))
 (segment (start 141.986 79.756) (end 141.986 88.011) (width 1) (layer F.Cu) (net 26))
 (segment (start 150.9395 70.8025) (end 141.986 79.756) (width 1) (layer F.Cu) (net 26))
 (segment (start 158.623 70.8025) (end 167.9575 70.8025) (width 1.25) (layer B.Cu) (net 26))
 (segment (start 144.526 89.01537) (end 144.526 88.011) (width 1) (layer B.Cu) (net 21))
 (segment (start 141.78387 91.7575) (end 144.526 89.01537) (width 1) (layer B.Cu) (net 21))
 (segment (start 140.6525 91.7575) (end 141.78387 91.7575) (width 1) (layer B.Cu) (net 21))
 (segment (start 158.623 75.946) (end 149.352 75.946) (width 1) (layer F.Cu) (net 21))
 (segment (start 144.526 80.772) (end 144.526 88.011) (width 1) (layer F.Cu) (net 21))
 (segment (start 149.352 75.946) (end 144.526 80.772) (width 1) (layer F.Cu) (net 21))
 (segment (start 167.9575 75.946) (end 158.623 75.946) (width 1.25) (layer B.Cu) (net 21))
 (segment (start 167.9575 91.2495) (end 167.9575 86.106) (width 1) (layer B.Cu) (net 2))
 (segment (start 158.623 86.106) (end 156.4005 86.106) (width 1.5) (layer B.Cu) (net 2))
 (segment (start 156.4005 86.106) (end 151.511 81.2165) (width 1.5) (layer B.Cu) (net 2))
 (segment (start 151.511 81.2165) (end 127.9525 81.2165) (width 1.5) (layer B.Cu) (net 2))
 (segment (start 114.6645 94.5045) (end 114.6645 103.378) (width 1.5) (layer B.Cu) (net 2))
 (segment (start 127.9525 81.2165) (end 114.6645 94.5045) (width 1.5) (layer B.Cu) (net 2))
 (segment (start 167.9575 91.2495) (end 166.1795 91.2495) (width 1.5) (layer B.Cu) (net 2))
 (segment (start 166.1795 91.2495) (end 162.3695 95.0595) (width 1.5) (layer B.Cu) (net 2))
 (segment (start 162.3695 102.964) (end 158.6535 106.68) (width 1.5) (layer B.Cu) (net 2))
 (segment (start 162.3695 95.0595) (end 162.3695 102.964) (width 1.5) (layer B.Cu) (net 2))
 (segment (start 158.623 86.106) (end 167.9575 86.106) (width 1.25) (layer B.Cu) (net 2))
 (segment (start 132.969 88.011) (end 132.969 89.027) (width 1) (layer B.Cu) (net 23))
 (segment (start 167.9575 96.3295) (end 167.9575 116.5225) (width 1) (layer B.Cu) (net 23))
 (segment (start 167.9575 116.5225) (end 166.1795 118.3005) (width 1) (layer B.Cu) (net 23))
 (segment (start 155.0035 118.3005) (end 151.5745 114.8715) (width 1) (layer B.Cu) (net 23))
 (segment (start 166.1795 118.3005) (end 155.0035 118.3005) (width 1) (layer B.Cu) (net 23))
 (segment (start 132.969 88.773) (end 132.969 88.011) (width 1) (layer B.Cu) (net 23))
 (segment (start 129.9845 91.7575) (end 132.969 88.773) (width 1) (layer B.Cu) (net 23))
 (segment (start 167.9575 96.3295) (end 163.195 96.3295) (width 1) (layer F.Cu) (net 23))
 (segment (start 149.9235 83.058) (end 132.969 83.058) (width 1) (layer B.Cu) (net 23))
 (segment (start 132.969 83.058) (end 132.969 83.058) (width 1) (layer B.Cu) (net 23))
 (via (at 132.969 83.058) (size 0.8) (drill 0.4) (layers F.Cu B.Cu) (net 23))
 (segment (start 132.969 88.011) (end 132.969 83.058) (width 1) (layer F.Cu) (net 23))
 (segment (start 149.9235 83.058) (end 152.654 85.7885) (width 1) (layer B.Cu) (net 23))
 (segment (start 152.654 85.7885) (end 153.289 86.4235) (width 1) (layer B.Cu) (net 23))
 (segment (start 153.289 86.4235) (end 153.289 86.4235) (width 1) (layer B.Cu) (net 23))
 (via (at 153.289 86.4235) (size 0.8) (drill 0.4) (layers F.Cu B.Cu) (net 23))
 (segment (start 163.195 96.3295) (end 153.289 86.4235) (width 1) (layer F.Cu) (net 23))
 (segment (start 136.3345 35.2425) (end 136.3345 61.4045) (width 1) (layer B.Cu) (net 4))
 (segment (start 136.3345 61.4045) (end 120.523 77.216) (width 1) (layer B.Cu) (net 4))
 (segment (start 107.7025 77.216) (end 104.4645 73.978) (width 1) (layer B.Cu) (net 4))
 (segment (start 120.523 77.216) (end 107.7025 77.216) (width 1) (layer B.Cu) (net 4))
 (segment (start 139.8905 102.9335) (end 142.113 102.9335) (width 1) (layer B.Cu) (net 19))
 (segment (start 139.3825 98.9965) (end 139.3825 102.4255) (width 1) (layer B.Cu) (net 19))
 (segment (start 139.3825 102.4255) (end 139.8905 102.9335) (width 1) (layer B.Cu) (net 19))
 (segment (start 135.509 95.123) (end 139.3825 98.9965) (width 1) (layer B.Cu) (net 19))
 (segment (start 135.509 88.011) (end 135.509 95.123) (width 1) (layer B.Cu) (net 19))
 (segment (start 145.3515 114.2365) (end 142.113 114.2365) (width 1) (layer B.Cu) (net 14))
 (segment (start 146.812 112.776) (end 145.3515 114.2365) (width 1) (layer B.Cu) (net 14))
 (segment (start 146.812 95.6945) (end 146.812 112.776) (width 1) (layer B.Cu) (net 14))
 (segment (start 150.114 92.3925) (end 146.812 95.6945) (width 1) (layer B.Cu) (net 14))
 (segment (start 150.114 91.059) (end 150.114 92.3925) (width 1) (layer B.Cu) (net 14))
 (segment (start 147.066 88.011) (end 150.114 91.059) (width 1) (layer B.Cu) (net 14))
 (segment (start 131.5085 97.8535) (end 130.048 96.393) (width 0.75) (layer B.Cu) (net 20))
 (segment (start 134.493 97.8535) (end 131.5085 97.8535) (width 0.75) (layer B.Cu) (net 20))
 (segment (start 142.113 97.8535) (end 141.478 97.8535) (width 1) (layer B.Cu) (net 16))
 (segment (start 142.113 97.8535) (end 141.6685 97.8535) (width 1) (layer B.Cu) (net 16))
 (segment (start 140.2715 97.8535) (end 142.113 97.8535) (width 1) (layer B.Cu) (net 16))
 (segment (start 137.6045 95.1865) (end 140.2715 97.8535) (width 1) (layer B.Cu) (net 16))
 (segment (start 137.6045 91.7575) (end 137.6045 95.1865) (width 1) (layer B.Cu) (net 16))
 (segment (start 131.953 109.1565) (end 130.048 107.2515) (width 0.75) (layer B.Cu) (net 15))
 (segment (start 134.493 109.1565) (end 131.953 109.1565) (width 0.75) (layer B.Cu) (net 15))
 (segment (start 142.113 109.1565) (end 142.8115 109.1565) (width 1) (layer B.Cu) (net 10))
 (segment (start 144.0815 109.1565) (end 142.113 109.1565) (width 1) (layer B.Cu) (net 10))
 (segment (start 145.288 107.95) (end 144.0815 109.1565) (width 1) (layer B.Cu) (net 10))
 (segment (start 145.288 94.742) (end 145.288 107.95) (width 1) (layer B.Cu) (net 10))
 (segment (start 148.2725 91.7575) (end 145.288 94.742) (width 1) (layer B.Cu) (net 10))
 (segment (start 119.888 73.9545) (end 119.8645 73.978) (width 1) (layer F.Cu) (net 1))
 (segment (start 133.7945 60.048) (end 119.8645 73.978) (width 1) (layer B.Cu) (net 1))
 (segment (start 133.7945 35.2425) (end 133.7945 60.048) (width 1) (layer B.Cu) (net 1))
 (segment (start 120.777 115.062) (end 121.9835 113.8555) (width 1) (layer B.Cu) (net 24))
 (segment (start 118.364 115.062) (end 120.777 115.062) (width 1) (layer B.Cu) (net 24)))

